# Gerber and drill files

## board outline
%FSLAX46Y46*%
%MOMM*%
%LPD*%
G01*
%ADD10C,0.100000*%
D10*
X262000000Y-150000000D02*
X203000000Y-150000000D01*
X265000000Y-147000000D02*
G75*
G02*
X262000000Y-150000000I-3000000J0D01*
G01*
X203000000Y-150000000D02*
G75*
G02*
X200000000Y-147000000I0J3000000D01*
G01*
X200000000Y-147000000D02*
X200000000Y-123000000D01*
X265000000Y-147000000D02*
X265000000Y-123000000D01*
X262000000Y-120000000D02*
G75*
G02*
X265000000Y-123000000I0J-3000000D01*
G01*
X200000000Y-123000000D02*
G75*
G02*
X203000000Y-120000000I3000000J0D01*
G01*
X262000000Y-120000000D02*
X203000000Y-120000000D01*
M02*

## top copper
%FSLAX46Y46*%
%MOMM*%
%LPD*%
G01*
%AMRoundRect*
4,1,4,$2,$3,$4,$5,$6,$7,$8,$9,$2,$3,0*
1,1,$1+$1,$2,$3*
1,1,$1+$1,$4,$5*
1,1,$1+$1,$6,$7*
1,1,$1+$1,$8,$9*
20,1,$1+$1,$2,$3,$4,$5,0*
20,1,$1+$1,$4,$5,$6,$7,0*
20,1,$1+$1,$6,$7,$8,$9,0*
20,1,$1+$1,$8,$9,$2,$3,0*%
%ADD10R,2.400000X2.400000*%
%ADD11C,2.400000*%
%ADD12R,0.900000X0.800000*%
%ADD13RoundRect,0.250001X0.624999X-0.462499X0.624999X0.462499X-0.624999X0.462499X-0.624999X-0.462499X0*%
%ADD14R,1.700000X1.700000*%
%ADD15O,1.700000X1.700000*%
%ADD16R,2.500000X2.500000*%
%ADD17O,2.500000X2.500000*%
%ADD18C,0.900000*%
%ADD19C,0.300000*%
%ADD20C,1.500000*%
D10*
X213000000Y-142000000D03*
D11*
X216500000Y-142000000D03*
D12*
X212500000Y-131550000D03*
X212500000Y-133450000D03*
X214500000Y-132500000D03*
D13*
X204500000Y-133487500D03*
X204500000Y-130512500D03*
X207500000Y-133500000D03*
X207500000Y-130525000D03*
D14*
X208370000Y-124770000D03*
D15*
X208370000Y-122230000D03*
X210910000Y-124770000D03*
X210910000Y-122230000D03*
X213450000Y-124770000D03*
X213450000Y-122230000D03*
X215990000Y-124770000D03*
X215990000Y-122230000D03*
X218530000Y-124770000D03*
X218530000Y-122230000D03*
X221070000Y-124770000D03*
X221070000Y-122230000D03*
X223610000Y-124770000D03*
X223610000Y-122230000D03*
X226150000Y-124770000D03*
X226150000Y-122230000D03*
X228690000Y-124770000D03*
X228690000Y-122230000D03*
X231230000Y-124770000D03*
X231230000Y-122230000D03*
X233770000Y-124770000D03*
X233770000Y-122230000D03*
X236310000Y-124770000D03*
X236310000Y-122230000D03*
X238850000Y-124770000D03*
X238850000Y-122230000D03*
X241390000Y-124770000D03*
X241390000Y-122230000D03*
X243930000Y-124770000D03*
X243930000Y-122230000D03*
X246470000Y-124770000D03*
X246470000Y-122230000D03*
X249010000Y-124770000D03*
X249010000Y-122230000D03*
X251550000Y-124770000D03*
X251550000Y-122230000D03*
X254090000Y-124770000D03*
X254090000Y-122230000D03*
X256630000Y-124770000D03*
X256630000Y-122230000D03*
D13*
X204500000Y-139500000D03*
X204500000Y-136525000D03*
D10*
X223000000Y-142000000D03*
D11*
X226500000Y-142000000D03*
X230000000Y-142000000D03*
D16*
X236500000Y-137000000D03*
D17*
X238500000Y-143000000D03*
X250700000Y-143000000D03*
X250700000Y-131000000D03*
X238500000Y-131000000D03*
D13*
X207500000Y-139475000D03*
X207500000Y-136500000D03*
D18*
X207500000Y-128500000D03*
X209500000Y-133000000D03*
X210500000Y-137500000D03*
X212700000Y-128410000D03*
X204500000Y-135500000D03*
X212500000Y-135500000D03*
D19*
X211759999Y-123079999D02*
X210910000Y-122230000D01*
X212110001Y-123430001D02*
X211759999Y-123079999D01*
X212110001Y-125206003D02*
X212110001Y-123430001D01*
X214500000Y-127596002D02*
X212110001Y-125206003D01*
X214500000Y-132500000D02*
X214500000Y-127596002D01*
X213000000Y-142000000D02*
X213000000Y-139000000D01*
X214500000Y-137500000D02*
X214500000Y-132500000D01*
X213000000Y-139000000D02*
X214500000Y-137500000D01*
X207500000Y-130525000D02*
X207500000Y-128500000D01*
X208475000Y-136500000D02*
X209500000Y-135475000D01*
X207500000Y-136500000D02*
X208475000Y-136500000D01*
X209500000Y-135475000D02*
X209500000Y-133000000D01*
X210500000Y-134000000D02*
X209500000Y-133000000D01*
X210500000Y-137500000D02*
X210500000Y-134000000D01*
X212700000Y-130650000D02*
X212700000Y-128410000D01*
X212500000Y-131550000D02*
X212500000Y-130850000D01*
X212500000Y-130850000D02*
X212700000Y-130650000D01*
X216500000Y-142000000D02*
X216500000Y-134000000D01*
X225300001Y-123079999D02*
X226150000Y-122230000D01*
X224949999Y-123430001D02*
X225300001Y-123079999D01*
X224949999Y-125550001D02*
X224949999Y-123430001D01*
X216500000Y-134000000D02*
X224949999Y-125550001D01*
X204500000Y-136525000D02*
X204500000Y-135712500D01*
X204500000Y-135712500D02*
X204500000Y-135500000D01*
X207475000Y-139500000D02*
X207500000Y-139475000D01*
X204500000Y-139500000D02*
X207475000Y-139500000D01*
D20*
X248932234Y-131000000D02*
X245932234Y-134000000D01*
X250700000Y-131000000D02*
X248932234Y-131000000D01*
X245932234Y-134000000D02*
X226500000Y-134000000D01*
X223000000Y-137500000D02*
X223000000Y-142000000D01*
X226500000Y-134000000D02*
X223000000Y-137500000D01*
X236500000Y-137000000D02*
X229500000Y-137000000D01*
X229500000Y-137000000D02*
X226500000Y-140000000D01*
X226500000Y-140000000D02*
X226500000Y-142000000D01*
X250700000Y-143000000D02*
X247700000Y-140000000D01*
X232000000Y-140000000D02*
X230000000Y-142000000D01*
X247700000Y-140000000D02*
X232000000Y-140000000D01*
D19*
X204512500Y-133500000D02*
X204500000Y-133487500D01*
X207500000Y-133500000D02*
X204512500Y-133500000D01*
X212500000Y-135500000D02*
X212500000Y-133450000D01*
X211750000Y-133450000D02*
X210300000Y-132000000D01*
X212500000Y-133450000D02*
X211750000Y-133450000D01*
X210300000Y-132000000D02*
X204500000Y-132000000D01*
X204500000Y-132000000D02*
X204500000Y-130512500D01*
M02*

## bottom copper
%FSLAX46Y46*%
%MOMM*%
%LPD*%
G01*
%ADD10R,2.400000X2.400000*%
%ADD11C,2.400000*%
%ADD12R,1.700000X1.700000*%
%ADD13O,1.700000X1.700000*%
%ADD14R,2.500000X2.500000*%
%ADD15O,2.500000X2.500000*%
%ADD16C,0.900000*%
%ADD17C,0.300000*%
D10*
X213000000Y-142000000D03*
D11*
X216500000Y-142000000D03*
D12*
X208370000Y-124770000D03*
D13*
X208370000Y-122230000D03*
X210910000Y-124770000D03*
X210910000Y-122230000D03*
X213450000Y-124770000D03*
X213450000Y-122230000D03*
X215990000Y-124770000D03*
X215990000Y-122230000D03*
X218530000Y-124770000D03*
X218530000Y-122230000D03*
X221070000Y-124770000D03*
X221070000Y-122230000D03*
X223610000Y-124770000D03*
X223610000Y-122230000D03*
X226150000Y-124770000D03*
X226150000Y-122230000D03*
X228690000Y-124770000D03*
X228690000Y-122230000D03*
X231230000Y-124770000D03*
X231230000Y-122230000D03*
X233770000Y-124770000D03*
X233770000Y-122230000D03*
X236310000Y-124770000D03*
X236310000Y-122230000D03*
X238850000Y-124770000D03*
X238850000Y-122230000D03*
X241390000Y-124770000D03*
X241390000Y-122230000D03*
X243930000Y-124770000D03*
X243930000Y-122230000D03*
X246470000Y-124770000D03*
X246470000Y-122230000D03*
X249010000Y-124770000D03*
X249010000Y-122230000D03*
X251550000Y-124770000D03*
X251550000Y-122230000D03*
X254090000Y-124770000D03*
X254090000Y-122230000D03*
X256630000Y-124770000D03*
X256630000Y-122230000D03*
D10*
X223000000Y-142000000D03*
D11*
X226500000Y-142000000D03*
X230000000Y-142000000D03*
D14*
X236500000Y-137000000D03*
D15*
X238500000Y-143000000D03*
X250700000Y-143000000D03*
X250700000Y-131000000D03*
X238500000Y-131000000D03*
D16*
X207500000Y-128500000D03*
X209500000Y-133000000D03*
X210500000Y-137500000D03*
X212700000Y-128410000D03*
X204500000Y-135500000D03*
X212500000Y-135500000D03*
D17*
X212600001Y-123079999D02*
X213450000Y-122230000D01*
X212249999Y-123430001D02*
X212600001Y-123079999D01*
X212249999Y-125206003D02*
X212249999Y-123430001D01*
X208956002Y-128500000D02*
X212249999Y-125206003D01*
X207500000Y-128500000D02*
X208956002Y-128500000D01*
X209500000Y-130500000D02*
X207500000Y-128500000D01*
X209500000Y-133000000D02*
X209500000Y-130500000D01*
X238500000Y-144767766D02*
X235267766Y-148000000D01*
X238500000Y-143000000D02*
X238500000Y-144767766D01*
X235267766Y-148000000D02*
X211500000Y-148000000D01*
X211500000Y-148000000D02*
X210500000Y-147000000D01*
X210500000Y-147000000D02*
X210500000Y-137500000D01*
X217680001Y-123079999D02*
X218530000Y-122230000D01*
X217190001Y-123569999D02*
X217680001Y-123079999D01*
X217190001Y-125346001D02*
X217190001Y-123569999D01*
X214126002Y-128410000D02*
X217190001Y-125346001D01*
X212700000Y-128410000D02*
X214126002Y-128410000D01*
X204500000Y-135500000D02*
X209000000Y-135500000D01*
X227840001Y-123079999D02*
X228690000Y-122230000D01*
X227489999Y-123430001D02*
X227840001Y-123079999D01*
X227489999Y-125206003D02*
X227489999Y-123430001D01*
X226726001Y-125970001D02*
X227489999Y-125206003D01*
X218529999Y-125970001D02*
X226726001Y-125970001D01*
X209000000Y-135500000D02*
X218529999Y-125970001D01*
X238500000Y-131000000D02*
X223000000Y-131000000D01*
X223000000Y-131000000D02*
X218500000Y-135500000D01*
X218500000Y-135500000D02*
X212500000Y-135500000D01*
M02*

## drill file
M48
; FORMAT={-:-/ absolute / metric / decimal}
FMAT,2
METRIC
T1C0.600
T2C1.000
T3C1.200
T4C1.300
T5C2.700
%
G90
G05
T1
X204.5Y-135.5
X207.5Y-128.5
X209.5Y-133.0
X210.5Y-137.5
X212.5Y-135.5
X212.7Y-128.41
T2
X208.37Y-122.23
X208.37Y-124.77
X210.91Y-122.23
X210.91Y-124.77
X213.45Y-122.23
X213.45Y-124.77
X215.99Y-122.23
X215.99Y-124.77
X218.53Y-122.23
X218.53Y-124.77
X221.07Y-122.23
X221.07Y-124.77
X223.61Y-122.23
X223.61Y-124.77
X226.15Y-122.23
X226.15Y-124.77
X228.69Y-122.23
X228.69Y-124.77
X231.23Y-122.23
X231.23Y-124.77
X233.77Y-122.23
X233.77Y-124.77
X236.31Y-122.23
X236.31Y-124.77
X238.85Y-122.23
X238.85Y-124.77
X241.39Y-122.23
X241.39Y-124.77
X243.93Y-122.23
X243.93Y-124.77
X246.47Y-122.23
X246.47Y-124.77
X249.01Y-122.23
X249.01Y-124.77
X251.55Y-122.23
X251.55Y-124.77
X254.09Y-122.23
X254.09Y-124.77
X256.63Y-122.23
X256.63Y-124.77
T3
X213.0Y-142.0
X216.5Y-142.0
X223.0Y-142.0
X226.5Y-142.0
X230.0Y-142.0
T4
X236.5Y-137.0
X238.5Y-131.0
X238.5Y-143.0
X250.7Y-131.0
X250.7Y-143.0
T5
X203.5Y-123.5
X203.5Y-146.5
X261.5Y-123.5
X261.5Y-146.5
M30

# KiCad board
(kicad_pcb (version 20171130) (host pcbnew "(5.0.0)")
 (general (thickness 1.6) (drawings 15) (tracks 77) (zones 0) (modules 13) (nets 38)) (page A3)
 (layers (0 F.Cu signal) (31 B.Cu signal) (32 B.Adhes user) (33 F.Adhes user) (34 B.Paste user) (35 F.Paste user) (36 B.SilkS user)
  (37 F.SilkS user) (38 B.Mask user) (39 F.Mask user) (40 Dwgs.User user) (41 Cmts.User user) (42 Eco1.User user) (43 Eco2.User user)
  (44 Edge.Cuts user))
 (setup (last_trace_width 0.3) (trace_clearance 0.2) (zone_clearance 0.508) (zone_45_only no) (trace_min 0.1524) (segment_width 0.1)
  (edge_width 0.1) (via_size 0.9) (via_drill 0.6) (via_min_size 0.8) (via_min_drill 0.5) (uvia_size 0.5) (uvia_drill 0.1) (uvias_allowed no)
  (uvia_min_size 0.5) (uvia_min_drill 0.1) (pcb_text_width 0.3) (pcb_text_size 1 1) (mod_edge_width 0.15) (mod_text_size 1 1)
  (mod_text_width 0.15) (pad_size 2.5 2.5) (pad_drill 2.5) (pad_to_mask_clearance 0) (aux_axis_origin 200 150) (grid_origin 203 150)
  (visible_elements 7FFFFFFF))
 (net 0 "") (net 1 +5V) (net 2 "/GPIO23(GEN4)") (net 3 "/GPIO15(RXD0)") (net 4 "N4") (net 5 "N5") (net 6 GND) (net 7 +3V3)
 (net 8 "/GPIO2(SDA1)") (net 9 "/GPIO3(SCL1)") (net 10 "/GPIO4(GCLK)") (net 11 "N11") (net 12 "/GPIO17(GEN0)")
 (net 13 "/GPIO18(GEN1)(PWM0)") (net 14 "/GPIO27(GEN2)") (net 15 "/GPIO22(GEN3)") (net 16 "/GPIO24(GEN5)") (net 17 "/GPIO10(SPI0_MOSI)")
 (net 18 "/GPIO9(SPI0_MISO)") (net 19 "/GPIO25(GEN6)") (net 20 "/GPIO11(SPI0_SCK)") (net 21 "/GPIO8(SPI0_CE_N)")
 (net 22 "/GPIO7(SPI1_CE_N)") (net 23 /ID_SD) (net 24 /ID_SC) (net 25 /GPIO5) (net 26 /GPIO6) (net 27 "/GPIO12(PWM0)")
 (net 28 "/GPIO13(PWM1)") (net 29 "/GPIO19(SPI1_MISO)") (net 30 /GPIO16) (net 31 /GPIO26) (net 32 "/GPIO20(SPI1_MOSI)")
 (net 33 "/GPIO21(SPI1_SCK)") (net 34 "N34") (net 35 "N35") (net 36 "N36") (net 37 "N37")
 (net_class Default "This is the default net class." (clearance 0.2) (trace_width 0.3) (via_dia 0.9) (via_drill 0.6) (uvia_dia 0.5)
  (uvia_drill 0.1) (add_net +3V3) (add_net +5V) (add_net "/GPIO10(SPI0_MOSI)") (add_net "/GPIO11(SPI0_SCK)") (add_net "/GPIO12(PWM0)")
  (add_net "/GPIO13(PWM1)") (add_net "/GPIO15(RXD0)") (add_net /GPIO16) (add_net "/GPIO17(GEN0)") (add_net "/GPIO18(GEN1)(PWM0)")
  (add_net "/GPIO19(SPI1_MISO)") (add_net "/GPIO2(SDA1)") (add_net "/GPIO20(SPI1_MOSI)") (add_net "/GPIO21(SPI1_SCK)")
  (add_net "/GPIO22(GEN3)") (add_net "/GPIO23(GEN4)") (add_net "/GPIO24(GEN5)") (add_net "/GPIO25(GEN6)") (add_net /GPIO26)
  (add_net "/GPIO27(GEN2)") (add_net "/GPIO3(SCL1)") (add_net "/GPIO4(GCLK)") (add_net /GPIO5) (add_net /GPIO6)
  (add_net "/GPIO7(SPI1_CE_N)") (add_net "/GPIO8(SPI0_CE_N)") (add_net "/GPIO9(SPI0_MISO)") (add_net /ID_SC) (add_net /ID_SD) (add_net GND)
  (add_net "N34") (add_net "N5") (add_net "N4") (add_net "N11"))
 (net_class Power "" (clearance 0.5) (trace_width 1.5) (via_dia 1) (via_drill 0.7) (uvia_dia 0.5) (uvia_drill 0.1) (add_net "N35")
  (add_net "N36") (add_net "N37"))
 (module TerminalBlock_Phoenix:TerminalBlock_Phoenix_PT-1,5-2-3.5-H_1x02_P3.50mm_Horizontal (layer F.Cu) (at 213 142)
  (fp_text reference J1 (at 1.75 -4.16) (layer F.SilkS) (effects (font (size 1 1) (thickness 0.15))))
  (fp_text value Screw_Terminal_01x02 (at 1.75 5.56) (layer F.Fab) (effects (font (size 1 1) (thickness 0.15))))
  (pad 1 thru_hole rect (at 0 0) (size 2.4 2.4) (drill 1.2) (layers *.Cu *.Mask) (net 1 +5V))
  (pad 2 thru_hole circle (at 3.5 0) (size 2.4 2.4) (drill 1.2) (layers *.Cu *.Mask) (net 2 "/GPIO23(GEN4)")))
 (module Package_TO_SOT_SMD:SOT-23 (layer F.Cu) (at 213.5 132.5)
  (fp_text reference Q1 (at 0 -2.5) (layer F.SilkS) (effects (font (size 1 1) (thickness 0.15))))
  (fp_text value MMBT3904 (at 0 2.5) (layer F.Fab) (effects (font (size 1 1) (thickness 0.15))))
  (pad 1 smd rect (at -1 -0.95) (size 0.9 0.8) (layers F.Cu F.Paste F.Mask) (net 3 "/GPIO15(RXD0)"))
  (pad 2 smd rect (at -1 0.95) (size 0.9 0.8) (layers F.Cu F.Paste F.Mask) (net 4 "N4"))
  (pad 3 smd rect (at 1 0) (size 0.9 0.8) (layers F.Cu F.Paste F.Mask) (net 1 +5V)))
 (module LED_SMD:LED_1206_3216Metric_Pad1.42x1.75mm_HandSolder (layer F.Cu) (at 204.5 132 90)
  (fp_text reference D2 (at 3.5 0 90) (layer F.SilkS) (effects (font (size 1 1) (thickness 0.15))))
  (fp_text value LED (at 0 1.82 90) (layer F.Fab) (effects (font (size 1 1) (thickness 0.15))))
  (pad 1 smd roundrect (at -1.4875 0 90) (size 1.425 1.75) (layers F.Cu F.Paste F.Mask) (roundrect_rratio 0.175439) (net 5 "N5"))
  (pad 2 smd roundrect (at 1.4875 0 90) (size 1.425 1.75) (layers F.Cu F.Paste F.Mask) (roundrect_rratio 0.175439) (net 4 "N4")))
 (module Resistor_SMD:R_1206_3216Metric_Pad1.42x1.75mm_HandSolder (layer F.Cu) (at 207.5 132.0125 90)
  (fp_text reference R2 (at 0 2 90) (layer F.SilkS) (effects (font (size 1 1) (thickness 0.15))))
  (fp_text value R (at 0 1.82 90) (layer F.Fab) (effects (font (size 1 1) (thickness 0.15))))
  (pad 1 smd roundrect (at -1.4875 0 90) (size 1.425 1.75) (layers F.Cu F.Paste F.Mask) (roundrect_rratio 0.175439) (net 5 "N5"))
  (pad 2 smd roundrect (at 1.4875 0 90) (size 1.425 1.75) (layers F.Cu F.Paste F.Mask) (roundrect_rratio 0.175439) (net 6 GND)))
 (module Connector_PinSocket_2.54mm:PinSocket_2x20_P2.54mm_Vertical (layer B.Cu) (at 208.37 124.77 270)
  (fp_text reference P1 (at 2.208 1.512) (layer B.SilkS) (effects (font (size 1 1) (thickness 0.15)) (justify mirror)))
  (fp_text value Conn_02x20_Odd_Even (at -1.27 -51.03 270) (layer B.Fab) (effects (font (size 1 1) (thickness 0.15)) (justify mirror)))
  (pad 1 thru_hole rect (at 0 0 270) (size 1.7 1.7) (drill 1) (layers *.Cu *.Mask) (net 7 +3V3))
  (pad 2 thru_hole oval (at -2.54 0 270) (size 1.7 1.7) (drill 1) (layers *.Cu *.Mask) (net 1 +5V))
  (pad 3 thru_hole oval (at 0 -2.54 270) (size 1.7 1.7) (drill 1) (layers *.Cu *.Mask) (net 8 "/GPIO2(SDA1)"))
  (pad 4 thru_hole oval (at -2.54 -2.54 270) (size 1.7 1.7) (drill 1) (layers *.Cu *.Mask) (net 1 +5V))
  (pad 5 thru_hole oval (at 0 -5.08 270) (size 1.7 1.7) (drill 1) (layers *.Cu *.Mask) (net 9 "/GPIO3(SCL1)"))
  (pad 6 thru_hole oval (at -2.54 -5.08 270) (size 1.7 1.7) (drill 1) (layers *.Cu *.Mask) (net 6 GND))
  (pad 7 thru_hole oval (at 0 -7.62 270) (size 1.7 1.7) (drill 1) (layers *.Cu *.Mask) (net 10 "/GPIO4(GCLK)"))
  (pad 8 thru_hole oval (at -2.54 -7.62 270) (size 1.7 1.7) (drill 1) (layers *.Cu *.Mask) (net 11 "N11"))
  (pad 9 thru_hole oval (at 0 -10.16 270) (size 1.7 1.7) (drill 1) (layers *.Cu *.Mask) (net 6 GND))
  (pad 10 thru_hole oval (at -2.54 -10.16 270) (size 1.7 1.7) (drill 1) (layers *.Cu *.Mask) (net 3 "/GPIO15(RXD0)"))
  (pad 11 thru_hole oval (at 0 -12.7 270) (size 1.7 1.7) (drill 1) (layers *.Cu *.Mask) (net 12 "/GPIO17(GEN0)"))
  (pad 12 thru_hole oval (at -2.54 -12.7 270) (size 1.7 1.7) (drill 1) (layers *.Cu *.Mask) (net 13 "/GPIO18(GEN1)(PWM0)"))
  (pad 13 thru_hole oval (at 0 -15.24 270) (size 1.7 1.7) (drill 1) (layers *.Cu *.Mask) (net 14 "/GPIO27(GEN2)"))
  (pad 14 thru_hole oval (at -2.54 -15.24 270) (size 1.7 1.7) (drill 1) (layers *.Cu *.Mask) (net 6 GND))
  (pad 15 thru_hole oval (at 0 -17.78 270) (size 1.7 1.7) (drill 1) (layers *.Cu *.Mask) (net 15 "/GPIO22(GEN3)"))
  (pad 16 thru_hole oval (at -2.54 -17.78 270) (size 1.7 1.7) (drill 1) (layers *.Cu *.Mask) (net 2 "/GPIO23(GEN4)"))
  (pad 17 thru_hole oval (at 0 -20.32 270) (size 1.7 1.7) (drill 1) (layers *.Cu *.Mask) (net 7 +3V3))
  (pad 18 thru_hole oval (at -2.54 -20.32 270) (size 1.7 1.7) (drill 1) (layers *.Cu *.Mask) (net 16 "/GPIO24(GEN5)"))
  (pad 19 thru_hole oval (at 0 -22.86 270) (size 1.7 1.7) (drill 1) (layers *.Cu *.Mask) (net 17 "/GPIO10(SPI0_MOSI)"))
  (pad 20 thru_hole oval (at -2.54 -22.86 270) (size 1.7 1.7) (drill 1) (layers *.Cu *.Mask) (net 6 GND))
  (pad 21 thru_hole oval (at 0 -25.4 270) (size 1.7 1.7) (drill 1) (layers *.Cu *.Mask) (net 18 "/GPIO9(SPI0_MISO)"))
  (pad 22 thru_hole oval (at -2.54 -25.4 270) (size 1.7 1.7) (drill 1) (layers *.Cu *.Mask) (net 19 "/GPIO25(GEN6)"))
  (pad 23 thru_hole oval (at 0 -27.94 270) (size 1.7 1.7) (drill 1) (layers *.Cu *.Mask) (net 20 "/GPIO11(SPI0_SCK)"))
  (pad 24 thru_hole oval (at -2.54 -27.94 270) (size 1.7 1.7) (drill 1) (layers *.Cu *.Mask) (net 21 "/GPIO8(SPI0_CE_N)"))
  (pad 25 thru_hole oval (at 0 -30.48 270) (size 1.7 1.7) (drill 1) (layers *.Cu *.Mask) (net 6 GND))
  (pad 26 thru_hole oval (at -2.54 -30.48 270) (size 1.7 1.7) (drill 1) (layers *.Cu *.Mask) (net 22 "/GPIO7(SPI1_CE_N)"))
  (pad 27 thru_hole oval (at 0 -33.02 270) (size 1.7 1.7) (drill 1) (layers *.Cu *.Mask) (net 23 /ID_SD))
  (pad 28 thru_hole oval (at -2.54 -33.02 270) (size 1.7 1.7) (drill 1) (layers *.Cu *.Mask) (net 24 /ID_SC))
  (pad 29 thru_hole oval (at 0 -35.56 270) (size 1.7 1.7) (drill 1) (layers *.Cu *.Mask) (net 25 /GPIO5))
  (pad 30 thru_hole oval (at -2.54 -35.56 270) (size 1.7 1.7) (drill 1) (layers *.Cu *.Mask) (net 6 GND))
  (pad 31 thru_hole oval (at 0 -38.1 270) (size 1.7 1.7) (drill 1) (layers *.Cu *.Mask) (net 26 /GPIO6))
  (pad 32 thru_hole oval (at -2.54 -38.1 270) (size 1.7 1.7) (drill 1) (layers *.Cu *.Mask) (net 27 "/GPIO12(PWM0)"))
  (pad 33 thru_hole oval (at 0 -40.64 270) (size 1.7 1.7) (drill 1) (layers *.Cu *.Mask) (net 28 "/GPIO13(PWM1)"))
  (pad 34 thru_hole oval (at -2.54 -40.64 270) (size 1.7 1.7) (drill 1) (layers *.Cu *.Mask) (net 6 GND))
  (pad 35 thru_hole oval (at 0 -43.18 270) (size 1.7 1.7) (drill 1) (layers *.Cu *.Mask) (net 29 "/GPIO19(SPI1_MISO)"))
  (pad 36 thru_hole oval (at -2.54 -43.18 270) (size 1.7 1.7) (drill 1) (layers *.Cu *.Mask) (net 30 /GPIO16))
  (pad 37 thru_hole oval (at 0 -45.72 270) (size 1.7 1.7) (drill 1) (layers *.Cu *.Mask) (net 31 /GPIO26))
  (pad 38 thru_hole oval (at -2.54 -45.72 270) (size 1.7 1.7) (drill 1) (layers *.Cu *.Mask) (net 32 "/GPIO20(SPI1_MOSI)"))
  (pad 39 thru_hole oval (at 0 -48.26 270) (size 1.7 1.7) (drill 1) (layers *.Cu *.Mask) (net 6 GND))
  (pad 40 thru_hole oval (at -2.54 -48.26 270) (size 1.7 1.7) (drill 1) (layers *.Cu *.Mask) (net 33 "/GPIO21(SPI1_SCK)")))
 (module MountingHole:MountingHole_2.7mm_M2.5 (layer F.Cu) (at 261.5 146.5)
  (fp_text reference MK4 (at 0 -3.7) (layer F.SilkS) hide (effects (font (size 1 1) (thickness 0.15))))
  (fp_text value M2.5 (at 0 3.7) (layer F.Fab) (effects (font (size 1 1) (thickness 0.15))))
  (pad 1 np_thru_hole circle (at 0 0) (size 2.7 2.7) (drill 2.7) (layers *.Cu *.Mask)))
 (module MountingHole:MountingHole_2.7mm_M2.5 (layer F.Cu) (at 203.5 146.5)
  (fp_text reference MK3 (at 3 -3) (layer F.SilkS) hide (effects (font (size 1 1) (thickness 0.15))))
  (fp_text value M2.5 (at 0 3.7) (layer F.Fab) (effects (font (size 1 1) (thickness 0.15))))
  (pad 1 np_thru_hole circle (at 0 0) (size 2.7 2.7) (drill 2.7) (layers *.Cu *.Mask)))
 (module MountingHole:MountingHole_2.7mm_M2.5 (layer F.Cu) (at 261.5 123.5 180)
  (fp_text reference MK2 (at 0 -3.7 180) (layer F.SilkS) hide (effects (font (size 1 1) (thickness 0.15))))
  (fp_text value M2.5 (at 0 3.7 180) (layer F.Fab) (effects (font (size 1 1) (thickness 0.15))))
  (pad 1 np_thru_hole circle (at 0 0 180) (size 2.7 2.7) (drill 2.7) (layers *.Cu *.Mask)))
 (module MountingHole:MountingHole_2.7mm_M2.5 (layer F.Cu) (at 203.5 123.5 180)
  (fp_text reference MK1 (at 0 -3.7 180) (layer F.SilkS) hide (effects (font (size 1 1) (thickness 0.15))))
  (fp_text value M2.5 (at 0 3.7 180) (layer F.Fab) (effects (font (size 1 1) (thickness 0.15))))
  (pad 1 np_thru_hole circle (at 0 0 180) (size 2.7 2.7) (drill 2.7) (layers *.Cu *.Mask)))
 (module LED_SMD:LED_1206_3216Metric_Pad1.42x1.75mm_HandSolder (layer F.Cu) (at 204.5 138.0125 90)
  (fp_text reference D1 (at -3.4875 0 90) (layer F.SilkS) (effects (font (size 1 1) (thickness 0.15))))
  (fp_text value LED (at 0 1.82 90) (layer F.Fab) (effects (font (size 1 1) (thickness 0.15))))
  (pad 1 smd roundrect (at -1.4875 0 90) (size 1.425 1.75) (layers F.Cu F.Paste F.Mask) (roundrect_rratio 0.175439) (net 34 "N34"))
  (pad 2 smd roundrect (at 1.4875 0 90) (size 1.425 1.75) (layers F.Cu F.Paste F.Mask) (roundrect_rratio 0.175439) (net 16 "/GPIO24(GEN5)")))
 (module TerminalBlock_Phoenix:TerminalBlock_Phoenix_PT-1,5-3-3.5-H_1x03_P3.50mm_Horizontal (layer F.Cu) (at 223 142)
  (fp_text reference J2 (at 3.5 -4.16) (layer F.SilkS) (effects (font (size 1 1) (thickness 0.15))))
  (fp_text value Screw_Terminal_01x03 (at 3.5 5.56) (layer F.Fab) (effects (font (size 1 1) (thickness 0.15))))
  (pad 1 thru_hole rect (at 0 0) (size 2.4 2.4) (drill 1.2) (layers *.Cu *.Mask) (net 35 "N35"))
  (pad 2 thru_hole circle (at 3.5 0) (size 2.4 2.4) (drill 1.2) (layers *.Cu *.Mask) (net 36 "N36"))
  (pad 3 thru_hole circle (at 7 0) (size 2.4 2.4) (drill 1.2) (layers *.Cu *.Mask) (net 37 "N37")))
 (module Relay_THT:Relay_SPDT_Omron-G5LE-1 (layer F.Cu) (at 236.5 137 90)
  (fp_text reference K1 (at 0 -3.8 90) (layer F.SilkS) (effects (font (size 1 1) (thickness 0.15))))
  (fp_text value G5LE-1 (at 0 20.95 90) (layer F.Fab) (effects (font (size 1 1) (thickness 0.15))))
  (pad 1 thru_hole rect (at 0 0 90) (size 2.5 2.5) (drill 1.3) (layers *.Cu *.Mask) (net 36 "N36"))
  (pad 2 thru_hole oval (at -6 2 90) (size 2.5 2.5) (drill 1.3) (layers *.Cu *.Mask) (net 6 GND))
  (pad 3 thru_hole oval (at -6 14.2 90) (size 2.5 2.5) (drill 1.3) (layers *.Cu *.Mask) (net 37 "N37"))
  (pad 4 thru_hole oval (at 6 14.2 90) (size 2.5 2.5) (drill 1.3) (layers *.Cu *.Mask) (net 35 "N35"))
  (pad 5 thru_hole oval (at 6 2 90) (size 2.5 2.5) (drill 1.3) (layers *.Cu *.Mask) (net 4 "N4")))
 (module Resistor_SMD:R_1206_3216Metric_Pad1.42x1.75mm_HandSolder (layer F.Cu) (at 207.5 137.9875 90)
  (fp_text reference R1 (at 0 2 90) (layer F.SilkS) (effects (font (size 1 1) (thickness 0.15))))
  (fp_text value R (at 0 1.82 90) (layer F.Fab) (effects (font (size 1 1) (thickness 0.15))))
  (pad 1 smd roundrect (at -1.4875 0 90) (size 1.425 1.75) (layers F.Cu F.Paste F.Mask) (roundrect_rratio 0.175439) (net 34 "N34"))
  (pad 2 smd roundrect (at 1.4875 0 90) (size 1.425 1.75) (layers F.Cu F.Paste F.Mask) (roundrect_rratio 0.175439) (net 6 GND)))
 (gr_line (start 262 150) (end 203 150) (layer Edge.Cuts) (width 0.1))
 (gr_arc (start 262 147) (end 262 150) (angle -90) (layer Edge.Cuts) (width 0.1))
 (gr_arc (start 203 147) (end 200 147) (angle -90) (layer Edge.Cuts) (width 0.1))
 (gr_line (start 200 147) (end 200 123) (layer Edge.Cuts) (width 0.1))
 (gr_line (start 265 147) (end 265 123) (layer Edge.Cuts) (width 0.1))
 (gr_arc (start 262 123) (end 262 120) (angle 90) (layer Edge.Cuts) (width 0.1))
 (gr_arc (start 203 123) (end 200 123) (angle 90) (layer Edge.Cuts) (width 0.1))
 (gr_line (start 262 120) (end 203 120) (layer Edge.Cuts) (width 0.1))
 (segment (start 211.759999 123.079999) (end 210.91 122.23) (width 0.3) (layer F.Cu) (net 1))
 (segment (start 212.110001 123.430001) (end 211.759999 123.079999) (width 0.3) (layer F.Cu) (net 1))
 (segment (start 212.110001 125.206003) (end 212.110001 123.430001) (width 0.3) (layer F.Cu) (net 1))
 (segment (start 214.5 127.596002) (end 212.110001 125.206003) (width 0.3) (layer F.Cu) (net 1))
 (segment (start 214.5 132.5) (end 214.5 127.596002) (width 0.3) (layer F.Cu) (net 1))
 (segment (start 213 142) (end 213 139) (width 0.3) (layer F.Cu) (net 1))
 (segment (start 214.5 137.5) (end 214.5 132.5) (width 0.3) (layer F.Cu) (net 1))
 (segment (start 213 139) (end 214.5 137.5) (width 0.3) (layer F.Cu) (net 1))
 (via (at 207.5 128.5) (size 0.9) (drill 0.6) (layers F.Cu B.Cu) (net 6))
 (segment (start 207.5 130.525) (end 207.5 128.5) (width 0.3) (layer F.Cu) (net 6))
 (segment (start 212.600001 123.079999) (end 213.45 122.23) (width 0.3) (layer B.Cu) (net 6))
 (segment (start 212.249999 123.430001) (end 212.600001 123.079999) (width 0.3) (layer B.Cu) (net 6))
 (segment (start 212.249999 125.206003) (end 212.249999 123.430001) (width 0.3) (layer B.Cu) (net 6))
 (segment (start 208.956002 128.5) (end 212.249999 125.206003) (width 0.3) (layer B.Cu) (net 6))
 (segment (start 207.5 128.5) (end 208.956002 128.5) (width 0.3) (layer B.Cu) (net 6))
 (segment (start 208.475 136.5) (end 209.5 135.475) (width 0.3) (layer F.Cu) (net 6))
 (segment (start 207.5 136.5) (end 208.475 136.5) (width 0.3) (layer F.Cu) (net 6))
 (via (at 209.5 133) (size 0.9) (drill 0.6) (layers F.Cu B.Cu) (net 6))
 (segment (start 209.5 135.475) (end 209.5 133) (width 0.3) (layer F.Cu) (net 6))
 (segment (start 209.5 130.5) (end 207.5 128.5) (width 0.3) (layer B.Cu) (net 6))
 (segment (start 209.5 133) (end 209.5 130.5) (width 0.3) (layer B.Cu) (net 6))
 (segment (start 238.5 144.767766) (end 235.267766 148) (width 0.3) (layer B.Cu) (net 6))
 (segment (start 238.5 143) (end 238.5 144.767766) (width 0.3) (layer B.Cu) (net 6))
 (segment (start 235.267766 148) (end 211.5 148) (width 0.3) (layer B.Cu) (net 6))
 (via (at 210.5 137.5) (size 0.9) (drill 0.6) (layers F.Cu B.Cu) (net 6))
 (segment (start 211.5 148) (end 210.5 147) (width 0.3) (layer B.Cu) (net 6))
 (segment (start 210.5 147) (end 210.5 137.5) (width 0.3) (layer B.Cu) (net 6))
 (segment (start 210.5 134) (end 209.5 133) (width 0.3) (layer F.Cu) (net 6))
 (segment (start 210.5 137.5) (end 210.5 134) (width 0.3) (layer F.Cu) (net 6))
 (via (at 212.7 128.41) (size 0.9) (drill 0.6) (layers F.Cu B.Cu) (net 3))
 (segment (start 212.7 130.65) (end 212.7 128.41) (width 0.3) (layer F.Cu) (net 3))
 (segment (start 212.5 131.55) (end 212.5 130.85) (width 0.3) (layer F.Cu) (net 3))
 (segment (start 212.5 130.85) (end 212.7 130.65) (width 0.3) (layer F.Cu) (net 3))
 (segment (start 217.680001 123.079999) (end 218.53 122.23) (width 0.3) (layer B.Cu) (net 3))
 (segment (start 217.190001 123.569999) (end 217.680001 123.079999) (width 0.3) (layer B.Cu) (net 3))
 (segment (start 217.190001 125.346001) (end 217.190001 123.569999) (width 0.3) (layer B.Cu) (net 3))
 (segment (start 214.126002 128.41) (end 217.190001 125.346001) (width 0.3) (layer B.Cu) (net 3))
 (segment (start 212.7 128.41) (end 214.126002 128.41) (width 0.3) (layer B.Cu) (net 3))
 (segment (start 216.5 142) (end 216.5 134) (width 0.3) (layer F.Cu) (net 2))
 (segment (start 225.300001 123.079999) (end 226.15 122.23) (width 0.3) (layer F.Cu) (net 2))
 (segment (start 224.949999 123.430001) (end 225.300001 123.079999) (width 0.3) (layer F.Cu) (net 2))
 (segment (start 224.949999 125.550001) (end 224.949999 123.430001) (width 0.3) (layer F.Cu) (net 2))
 (segment (start 216.5 134) (end 224.949999 125.550001) (width 0.3) (layer F.Cu) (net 2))
 (segment (start 204.5 136.525) (end 204.5 135.7125) (width 0.3) (layer F.Cu) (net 16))
 (via (at 204.5 135.5) (size 0.9) (drill 0.6) (layers F.Cu B.Cu) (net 16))
 (segment (start 204.5 135.7125) (end 204.5 135.5) (width 0.3) (layer F.Cu) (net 16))
 (segment (start 204.5 135.5) (end 209 135.5) (width 0.3) (layer B.Cu) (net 16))
 (segment (start 227.840001 123.079999) (end 228.69 122.23) (width 0.3) (layer B.Cu) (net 16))
 (segment (start 227.489999 123.430001) (end 227.840001 123.079999) (width 0.3) (layer B.Cu) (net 16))
 (segment (start 227.489999 125.206003) (end 227.489999 123.430001) (width 0.3) (layer B.Cu) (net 16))
 (segment (start 226.726001 125.970001) (end 227.489999 125.206003) (width 0.3) (layer B.Cu) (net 16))
 (segment (start 218.529999 125.970001) (end 226.726001 125.970001) (width 0.3) (layer B.Cu) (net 16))
 (segment (start 209 135.5) (end 218.529999 125.970001) (width 0.3) (layer B.Cu) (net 16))
 (segment (start 207.475 139.5) (end 207.5 139.475) (width 0.3) (layer F.Cu) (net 34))
 (segment (start 204.5 139.5) (end 207.475 139.5) (width 0.3) (layer F.Cu) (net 34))
 (segment (start 248.932234 131) (end 245.932234 134) (width 1.5) (layer F.Cu) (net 35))
 (segment (start 250.7 131) (end 248.932234 131) (width 1.5) (layer F.Cu) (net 35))
 (segment (start 245.932234 134) (end 226.5 134) (width 1.5) (layer F.Cu) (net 35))
 (segment (start 223 137.5) (end 223 142) (width 1.5) (layer F.Cu) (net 35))
 (segment (start 226.5 134) (end 223 137.5) (width 1.5) (layer F.Cu) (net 35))
 (segment (start 236.5 137) (end 229.5 137) (width 1.5) (layer F.Cu) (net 36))
 (segment (start 229.5 137) (end 226.5 140) (width 1.5) (layer F.Cu) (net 36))
 (segment (start 226.5 140) (end 226.5 142) (width 1.5) (layer F.Cu) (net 36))
 (segment (start 250.7 143) (end 247.7 140) (width 1.5) (layer F.Cu) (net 37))
 (segment (start 232 140) (end 230 142) (width 1.5) (layer F.Cu) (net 37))
 (segment (start 247.7 140) (end 232 140) (width 1.5) (layer F.Cu) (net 37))
 (segment (start 204.5125 133.5) (end 204.5 133.4875) (width 0.3) (layer F.Cu) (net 5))
 (segment (start 207.5 133.5) (end 204.5125 133.5) (width 0.3) (layer F.Cu) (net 5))
 (segment (start 238.5 131) (end 223 131) (width 0.3) (layer B.Cu) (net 4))
 (segment (start 223 131) (end 218.5 135.5) (width 0.3) (layer B.Cu) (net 4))
 (via (at 212.5 135.5) (size 0.9) (drill 0.6) (layers F.Cu B.Cu) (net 4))
 (segment (start 218.5 135.5) (end 212.5 135.5) (width 0.3) (layer B.Cu) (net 4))
 (segment (start 212.5 135.5) (end 212.5 133.45) (width 0.3) (layer F.Cu) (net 4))
 (segment (start 211.75 133.45) (end 210.3 132) (width 0.3) (layer F.Cu) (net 4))
 (segment (start 212.5 133.45) (end 211.75 133.45) (width 0.3) (layer F.Cu) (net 4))
 (segment (start 210.3 132) (end 204.5 132) (width 0.3) (layer F.Cu) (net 4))
 (segment (start 204.5 132) (end 204.5 130.5125) (width 0.3) (layer F.Cu) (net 4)))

